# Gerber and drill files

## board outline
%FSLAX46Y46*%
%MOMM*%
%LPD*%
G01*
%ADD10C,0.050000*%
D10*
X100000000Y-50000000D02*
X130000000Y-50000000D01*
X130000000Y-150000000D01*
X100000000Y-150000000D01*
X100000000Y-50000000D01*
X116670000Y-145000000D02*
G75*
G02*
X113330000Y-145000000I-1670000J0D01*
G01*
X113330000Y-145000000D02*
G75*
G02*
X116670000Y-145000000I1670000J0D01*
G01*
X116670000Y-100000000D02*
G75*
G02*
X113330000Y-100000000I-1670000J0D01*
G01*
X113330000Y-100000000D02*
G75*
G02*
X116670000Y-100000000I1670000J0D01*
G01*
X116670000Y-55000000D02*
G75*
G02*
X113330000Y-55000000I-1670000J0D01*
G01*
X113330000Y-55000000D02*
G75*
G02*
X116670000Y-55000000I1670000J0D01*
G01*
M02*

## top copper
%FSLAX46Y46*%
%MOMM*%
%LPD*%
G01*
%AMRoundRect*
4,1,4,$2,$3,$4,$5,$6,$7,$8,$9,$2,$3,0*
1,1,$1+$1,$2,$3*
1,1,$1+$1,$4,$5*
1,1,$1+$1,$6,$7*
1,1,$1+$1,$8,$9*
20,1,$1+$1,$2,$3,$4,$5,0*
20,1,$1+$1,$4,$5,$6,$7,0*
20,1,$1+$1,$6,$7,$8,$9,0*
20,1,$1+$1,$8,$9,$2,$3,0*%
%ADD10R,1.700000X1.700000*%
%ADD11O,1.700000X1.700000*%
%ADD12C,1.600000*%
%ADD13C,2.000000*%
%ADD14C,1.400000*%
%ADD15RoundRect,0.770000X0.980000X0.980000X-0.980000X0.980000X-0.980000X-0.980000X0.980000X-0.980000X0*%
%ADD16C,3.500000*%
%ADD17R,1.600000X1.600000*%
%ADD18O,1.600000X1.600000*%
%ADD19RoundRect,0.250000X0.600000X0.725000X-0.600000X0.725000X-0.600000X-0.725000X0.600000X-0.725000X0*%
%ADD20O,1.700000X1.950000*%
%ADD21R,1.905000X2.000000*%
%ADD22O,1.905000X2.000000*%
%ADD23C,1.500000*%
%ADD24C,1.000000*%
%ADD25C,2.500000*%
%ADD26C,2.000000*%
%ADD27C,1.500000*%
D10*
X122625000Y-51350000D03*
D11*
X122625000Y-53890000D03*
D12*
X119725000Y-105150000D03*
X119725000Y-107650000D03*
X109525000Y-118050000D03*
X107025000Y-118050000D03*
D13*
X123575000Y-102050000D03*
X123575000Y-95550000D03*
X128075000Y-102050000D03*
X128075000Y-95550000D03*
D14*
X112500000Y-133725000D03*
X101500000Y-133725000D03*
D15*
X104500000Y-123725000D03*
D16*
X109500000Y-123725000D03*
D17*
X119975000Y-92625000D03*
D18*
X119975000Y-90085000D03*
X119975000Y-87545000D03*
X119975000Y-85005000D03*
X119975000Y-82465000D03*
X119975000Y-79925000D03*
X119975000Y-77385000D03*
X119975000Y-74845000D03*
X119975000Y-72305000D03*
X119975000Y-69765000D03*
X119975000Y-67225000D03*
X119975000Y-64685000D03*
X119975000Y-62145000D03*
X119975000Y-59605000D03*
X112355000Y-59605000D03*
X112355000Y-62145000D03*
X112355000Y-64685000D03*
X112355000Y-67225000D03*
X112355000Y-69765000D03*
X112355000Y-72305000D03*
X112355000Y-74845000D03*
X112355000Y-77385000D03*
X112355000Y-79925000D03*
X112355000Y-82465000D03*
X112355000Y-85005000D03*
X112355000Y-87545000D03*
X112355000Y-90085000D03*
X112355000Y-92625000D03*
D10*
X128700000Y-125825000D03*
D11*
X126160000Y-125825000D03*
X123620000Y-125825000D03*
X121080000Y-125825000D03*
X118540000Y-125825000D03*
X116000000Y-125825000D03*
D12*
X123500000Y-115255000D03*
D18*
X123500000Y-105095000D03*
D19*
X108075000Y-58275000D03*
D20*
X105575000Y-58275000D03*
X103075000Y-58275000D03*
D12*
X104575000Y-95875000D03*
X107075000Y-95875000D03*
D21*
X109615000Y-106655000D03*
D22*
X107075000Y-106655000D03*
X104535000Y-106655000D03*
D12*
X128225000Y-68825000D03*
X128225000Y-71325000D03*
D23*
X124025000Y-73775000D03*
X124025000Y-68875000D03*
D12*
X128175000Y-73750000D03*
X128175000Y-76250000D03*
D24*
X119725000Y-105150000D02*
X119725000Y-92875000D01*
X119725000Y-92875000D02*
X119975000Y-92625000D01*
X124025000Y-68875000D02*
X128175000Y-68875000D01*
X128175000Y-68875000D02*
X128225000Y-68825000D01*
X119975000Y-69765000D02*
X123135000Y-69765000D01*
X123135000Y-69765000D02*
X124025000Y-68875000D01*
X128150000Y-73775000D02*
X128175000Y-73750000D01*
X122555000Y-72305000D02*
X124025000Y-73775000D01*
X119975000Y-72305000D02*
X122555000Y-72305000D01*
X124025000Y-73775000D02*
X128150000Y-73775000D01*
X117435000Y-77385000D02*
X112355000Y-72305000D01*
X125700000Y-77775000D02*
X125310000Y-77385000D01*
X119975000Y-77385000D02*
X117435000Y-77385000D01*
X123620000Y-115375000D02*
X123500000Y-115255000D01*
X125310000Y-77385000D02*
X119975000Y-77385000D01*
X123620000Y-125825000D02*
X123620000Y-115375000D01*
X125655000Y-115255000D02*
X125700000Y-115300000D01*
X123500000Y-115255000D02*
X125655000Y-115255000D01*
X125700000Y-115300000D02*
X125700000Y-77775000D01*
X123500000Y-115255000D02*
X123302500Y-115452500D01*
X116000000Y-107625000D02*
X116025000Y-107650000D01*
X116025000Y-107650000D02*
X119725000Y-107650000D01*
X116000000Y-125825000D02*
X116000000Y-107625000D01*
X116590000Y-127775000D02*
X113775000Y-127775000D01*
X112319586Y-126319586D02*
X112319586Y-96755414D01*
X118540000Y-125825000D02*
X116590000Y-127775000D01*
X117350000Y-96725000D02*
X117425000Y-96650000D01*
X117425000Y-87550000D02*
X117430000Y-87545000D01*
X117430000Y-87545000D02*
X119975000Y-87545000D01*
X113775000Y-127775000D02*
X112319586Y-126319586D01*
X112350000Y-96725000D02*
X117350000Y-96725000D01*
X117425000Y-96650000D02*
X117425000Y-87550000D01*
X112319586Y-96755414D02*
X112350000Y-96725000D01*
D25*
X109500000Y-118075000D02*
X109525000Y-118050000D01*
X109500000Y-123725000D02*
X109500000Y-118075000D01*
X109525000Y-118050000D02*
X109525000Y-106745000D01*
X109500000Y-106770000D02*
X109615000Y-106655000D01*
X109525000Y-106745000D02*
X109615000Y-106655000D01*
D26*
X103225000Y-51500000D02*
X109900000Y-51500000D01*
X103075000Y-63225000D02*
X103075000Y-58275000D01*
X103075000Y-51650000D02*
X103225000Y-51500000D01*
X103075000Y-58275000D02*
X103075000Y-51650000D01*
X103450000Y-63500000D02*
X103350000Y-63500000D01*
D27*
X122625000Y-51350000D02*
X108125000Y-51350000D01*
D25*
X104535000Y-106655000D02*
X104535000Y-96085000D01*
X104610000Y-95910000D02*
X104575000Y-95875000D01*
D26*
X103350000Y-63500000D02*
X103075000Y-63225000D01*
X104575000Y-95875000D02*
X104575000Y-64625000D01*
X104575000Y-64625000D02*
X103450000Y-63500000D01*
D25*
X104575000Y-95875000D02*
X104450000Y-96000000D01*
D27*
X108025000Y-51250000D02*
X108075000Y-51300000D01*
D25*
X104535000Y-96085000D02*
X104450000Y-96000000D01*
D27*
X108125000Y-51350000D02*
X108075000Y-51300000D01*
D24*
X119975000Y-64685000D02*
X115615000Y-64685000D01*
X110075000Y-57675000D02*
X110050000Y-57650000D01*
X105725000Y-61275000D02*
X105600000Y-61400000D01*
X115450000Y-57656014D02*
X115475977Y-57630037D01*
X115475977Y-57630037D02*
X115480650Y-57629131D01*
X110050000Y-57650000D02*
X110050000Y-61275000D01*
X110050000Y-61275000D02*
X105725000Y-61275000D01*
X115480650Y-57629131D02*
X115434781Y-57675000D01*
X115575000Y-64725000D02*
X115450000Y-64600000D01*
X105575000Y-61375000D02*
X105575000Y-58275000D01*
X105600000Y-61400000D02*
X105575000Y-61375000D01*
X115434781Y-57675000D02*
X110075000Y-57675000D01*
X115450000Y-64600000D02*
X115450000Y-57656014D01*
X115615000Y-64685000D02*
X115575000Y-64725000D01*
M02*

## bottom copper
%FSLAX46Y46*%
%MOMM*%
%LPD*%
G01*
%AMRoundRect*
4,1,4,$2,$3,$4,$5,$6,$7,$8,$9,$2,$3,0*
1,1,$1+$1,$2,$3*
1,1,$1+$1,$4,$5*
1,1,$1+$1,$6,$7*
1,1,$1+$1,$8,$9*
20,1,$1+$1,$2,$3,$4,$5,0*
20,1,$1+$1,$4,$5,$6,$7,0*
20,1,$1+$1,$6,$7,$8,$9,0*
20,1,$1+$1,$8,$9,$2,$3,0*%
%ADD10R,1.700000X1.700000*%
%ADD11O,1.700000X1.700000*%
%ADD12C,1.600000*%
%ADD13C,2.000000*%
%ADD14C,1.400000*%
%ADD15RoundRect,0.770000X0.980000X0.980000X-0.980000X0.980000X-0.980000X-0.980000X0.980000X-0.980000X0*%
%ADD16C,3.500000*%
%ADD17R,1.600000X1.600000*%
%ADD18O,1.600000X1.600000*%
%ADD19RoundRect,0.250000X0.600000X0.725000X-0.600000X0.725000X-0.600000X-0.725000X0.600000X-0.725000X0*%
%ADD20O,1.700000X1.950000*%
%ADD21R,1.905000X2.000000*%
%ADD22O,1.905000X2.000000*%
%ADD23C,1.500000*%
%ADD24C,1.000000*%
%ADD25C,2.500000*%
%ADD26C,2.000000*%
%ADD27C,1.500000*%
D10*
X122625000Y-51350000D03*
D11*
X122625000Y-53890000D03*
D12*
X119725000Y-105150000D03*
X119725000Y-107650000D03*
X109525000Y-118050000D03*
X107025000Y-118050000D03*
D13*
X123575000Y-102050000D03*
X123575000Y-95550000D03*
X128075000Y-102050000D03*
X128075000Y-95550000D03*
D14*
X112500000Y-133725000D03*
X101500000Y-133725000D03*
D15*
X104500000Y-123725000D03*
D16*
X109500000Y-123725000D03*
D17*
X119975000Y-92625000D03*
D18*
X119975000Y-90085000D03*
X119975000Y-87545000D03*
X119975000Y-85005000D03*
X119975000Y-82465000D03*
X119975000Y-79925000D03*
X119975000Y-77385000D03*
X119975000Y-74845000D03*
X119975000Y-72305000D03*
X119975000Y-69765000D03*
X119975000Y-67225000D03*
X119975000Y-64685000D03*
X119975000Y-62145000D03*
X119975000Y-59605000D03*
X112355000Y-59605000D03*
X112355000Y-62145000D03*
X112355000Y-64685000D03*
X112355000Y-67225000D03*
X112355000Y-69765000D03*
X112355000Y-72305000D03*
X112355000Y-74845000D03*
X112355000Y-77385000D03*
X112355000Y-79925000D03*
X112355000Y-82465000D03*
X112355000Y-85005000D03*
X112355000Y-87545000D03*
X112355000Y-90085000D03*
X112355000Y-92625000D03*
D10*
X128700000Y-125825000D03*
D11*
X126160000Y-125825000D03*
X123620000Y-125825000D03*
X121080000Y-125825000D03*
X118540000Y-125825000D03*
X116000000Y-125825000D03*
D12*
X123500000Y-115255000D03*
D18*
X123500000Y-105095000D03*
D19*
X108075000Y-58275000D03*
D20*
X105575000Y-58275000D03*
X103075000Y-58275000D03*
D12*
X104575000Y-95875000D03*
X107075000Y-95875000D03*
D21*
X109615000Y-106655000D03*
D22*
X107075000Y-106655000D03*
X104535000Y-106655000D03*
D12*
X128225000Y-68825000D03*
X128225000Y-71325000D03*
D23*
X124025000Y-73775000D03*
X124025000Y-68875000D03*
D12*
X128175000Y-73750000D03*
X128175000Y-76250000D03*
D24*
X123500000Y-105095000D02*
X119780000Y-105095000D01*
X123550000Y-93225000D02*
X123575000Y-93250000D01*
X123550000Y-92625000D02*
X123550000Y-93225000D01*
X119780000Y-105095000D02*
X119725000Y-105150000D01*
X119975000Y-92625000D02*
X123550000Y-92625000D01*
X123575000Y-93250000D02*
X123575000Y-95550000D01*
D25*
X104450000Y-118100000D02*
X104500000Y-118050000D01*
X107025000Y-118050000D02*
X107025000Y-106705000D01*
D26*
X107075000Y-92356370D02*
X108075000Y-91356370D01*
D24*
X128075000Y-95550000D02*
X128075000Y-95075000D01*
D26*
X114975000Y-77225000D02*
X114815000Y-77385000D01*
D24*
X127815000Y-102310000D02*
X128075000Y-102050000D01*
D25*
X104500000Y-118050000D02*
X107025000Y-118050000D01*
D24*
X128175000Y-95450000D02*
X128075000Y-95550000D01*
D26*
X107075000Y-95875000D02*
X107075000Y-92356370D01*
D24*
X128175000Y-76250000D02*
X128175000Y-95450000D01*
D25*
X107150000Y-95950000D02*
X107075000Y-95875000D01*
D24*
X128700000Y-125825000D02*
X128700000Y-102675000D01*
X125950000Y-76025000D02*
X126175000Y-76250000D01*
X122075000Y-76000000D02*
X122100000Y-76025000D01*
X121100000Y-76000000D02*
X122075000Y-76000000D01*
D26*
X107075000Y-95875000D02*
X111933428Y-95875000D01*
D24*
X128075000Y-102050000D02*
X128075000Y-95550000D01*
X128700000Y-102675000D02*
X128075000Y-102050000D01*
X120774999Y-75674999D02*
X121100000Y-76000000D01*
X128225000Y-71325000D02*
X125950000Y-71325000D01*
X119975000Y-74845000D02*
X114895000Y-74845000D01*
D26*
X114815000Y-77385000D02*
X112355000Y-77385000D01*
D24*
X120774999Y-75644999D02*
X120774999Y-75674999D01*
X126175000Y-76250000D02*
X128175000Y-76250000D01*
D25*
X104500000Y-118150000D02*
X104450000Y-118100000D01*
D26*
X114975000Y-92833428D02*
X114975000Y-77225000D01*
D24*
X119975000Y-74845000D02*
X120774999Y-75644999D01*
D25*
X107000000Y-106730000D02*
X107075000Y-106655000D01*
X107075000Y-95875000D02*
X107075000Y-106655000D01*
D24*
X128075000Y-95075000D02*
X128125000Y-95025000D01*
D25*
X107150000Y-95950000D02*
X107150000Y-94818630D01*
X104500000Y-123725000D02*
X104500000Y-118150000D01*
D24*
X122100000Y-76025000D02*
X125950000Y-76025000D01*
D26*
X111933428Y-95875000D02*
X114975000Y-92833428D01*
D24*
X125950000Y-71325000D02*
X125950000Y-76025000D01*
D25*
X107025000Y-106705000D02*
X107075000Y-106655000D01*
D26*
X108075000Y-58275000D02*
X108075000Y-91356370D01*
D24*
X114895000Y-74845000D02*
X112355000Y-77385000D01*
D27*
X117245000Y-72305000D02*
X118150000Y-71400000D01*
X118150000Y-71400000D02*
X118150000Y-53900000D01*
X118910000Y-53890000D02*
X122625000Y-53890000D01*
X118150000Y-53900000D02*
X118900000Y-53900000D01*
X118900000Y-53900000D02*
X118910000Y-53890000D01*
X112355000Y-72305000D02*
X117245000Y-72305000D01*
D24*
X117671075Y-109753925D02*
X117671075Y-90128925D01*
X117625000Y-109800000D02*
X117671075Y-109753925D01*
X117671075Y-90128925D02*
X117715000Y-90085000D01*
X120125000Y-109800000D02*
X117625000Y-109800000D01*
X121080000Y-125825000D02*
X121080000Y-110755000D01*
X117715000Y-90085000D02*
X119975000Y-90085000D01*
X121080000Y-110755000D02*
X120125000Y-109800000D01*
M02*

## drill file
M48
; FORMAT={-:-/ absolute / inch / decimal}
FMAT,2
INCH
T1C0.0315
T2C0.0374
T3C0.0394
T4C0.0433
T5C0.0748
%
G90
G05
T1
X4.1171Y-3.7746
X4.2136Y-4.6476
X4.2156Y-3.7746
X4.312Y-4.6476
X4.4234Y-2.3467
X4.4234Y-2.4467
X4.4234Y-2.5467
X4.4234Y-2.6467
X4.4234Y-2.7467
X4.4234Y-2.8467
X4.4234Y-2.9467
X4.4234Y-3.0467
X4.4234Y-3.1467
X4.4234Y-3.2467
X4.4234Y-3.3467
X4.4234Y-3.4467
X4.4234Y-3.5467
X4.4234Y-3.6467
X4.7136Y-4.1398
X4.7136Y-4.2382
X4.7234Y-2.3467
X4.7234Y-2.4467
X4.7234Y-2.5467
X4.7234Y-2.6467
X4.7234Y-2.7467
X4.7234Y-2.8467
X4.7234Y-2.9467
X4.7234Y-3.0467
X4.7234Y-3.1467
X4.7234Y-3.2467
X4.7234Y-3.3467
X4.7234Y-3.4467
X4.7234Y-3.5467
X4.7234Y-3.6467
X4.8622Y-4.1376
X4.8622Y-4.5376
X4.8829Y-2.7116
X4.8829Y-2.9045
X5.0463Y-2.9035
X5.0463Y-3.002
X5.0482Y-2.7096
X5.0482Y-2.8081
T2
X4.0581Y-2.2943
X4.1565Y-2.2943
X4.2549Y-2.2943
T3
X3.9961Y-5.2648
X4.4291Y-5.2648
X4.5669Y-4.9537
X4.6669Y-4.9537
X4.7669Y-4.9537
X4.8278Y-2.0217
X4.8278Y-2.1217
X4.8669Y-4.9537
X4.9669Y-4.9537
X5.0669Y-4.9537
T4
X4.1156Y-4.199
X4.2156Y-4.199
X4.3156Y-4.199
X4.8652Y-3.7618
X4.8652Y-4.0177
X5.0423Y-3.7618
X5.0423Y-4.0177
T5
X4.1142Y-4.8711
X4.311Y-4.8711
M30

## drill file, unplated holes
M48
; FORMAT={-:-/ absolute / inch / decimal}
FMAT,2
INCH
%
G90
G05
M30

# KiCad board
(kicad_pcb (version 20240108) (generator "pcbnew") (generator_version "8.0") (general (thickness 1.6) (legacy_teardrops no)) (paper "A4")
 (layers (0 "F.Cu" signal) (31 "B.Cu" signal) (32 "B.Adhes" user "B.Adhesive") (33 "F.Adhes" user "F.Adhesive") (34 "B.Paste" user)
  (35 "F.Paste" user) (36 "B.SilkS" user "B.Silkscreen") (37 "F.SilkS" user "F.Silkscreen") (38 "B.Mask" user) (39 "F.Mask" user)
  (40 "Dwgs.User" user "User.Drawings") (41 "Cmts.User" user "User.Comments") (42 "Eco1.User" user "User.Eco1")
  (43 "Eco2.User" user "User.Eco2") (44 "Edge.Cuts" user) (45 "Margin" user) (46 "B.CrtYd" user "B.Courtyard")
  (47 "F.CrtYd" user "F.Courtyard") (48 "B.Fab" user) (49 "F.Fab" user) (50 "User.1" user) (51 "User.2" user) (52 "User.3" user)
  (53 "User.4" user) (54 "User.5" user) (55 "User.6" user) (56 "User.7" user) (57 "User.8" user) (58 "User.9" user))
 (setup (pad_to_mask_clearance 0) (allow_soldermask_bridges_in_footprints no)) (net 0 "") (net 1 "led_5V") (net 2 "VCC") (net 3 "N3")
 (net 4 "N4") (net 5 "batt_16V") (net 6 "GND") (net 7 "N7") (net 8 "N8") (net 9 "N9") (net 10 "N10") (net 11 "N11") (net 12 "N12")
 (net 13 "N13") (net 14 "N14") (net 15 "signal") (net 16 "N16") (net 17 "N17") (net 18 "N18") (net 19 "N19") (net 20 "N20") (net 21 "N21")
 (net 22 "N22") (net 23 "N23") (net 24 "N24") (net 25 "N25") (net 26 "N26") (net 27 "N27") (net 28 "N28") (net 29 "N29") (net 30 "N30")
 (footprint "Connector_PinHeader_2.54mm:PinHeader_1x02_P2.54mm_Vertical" (layer "F.Cu") (at 122.625 51.35)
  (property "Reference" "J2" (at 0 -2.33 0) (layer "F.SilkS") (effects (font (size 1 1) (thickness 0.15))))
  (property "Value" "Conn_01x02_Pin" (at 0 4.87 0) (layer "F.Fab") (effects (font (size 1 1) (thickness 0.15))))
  (pad "1" thru_hole rect (at 0 0) (size 1.7 1.7) (drill 1) (layers "*.Cu" "*.Mask") (remove_unused_layers no) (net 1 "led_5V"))
  (pad "2" thru_hole oval (at 0 2.54) (size 1.7 1.7) (drill 1) (layers "*.Cu" "*.Mask") (remove_unused_layers no) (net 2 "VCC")))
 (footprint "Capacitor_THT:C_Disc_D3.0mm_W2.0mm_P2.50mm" (layer "F.Cu") (at 119.725 105.15 -90)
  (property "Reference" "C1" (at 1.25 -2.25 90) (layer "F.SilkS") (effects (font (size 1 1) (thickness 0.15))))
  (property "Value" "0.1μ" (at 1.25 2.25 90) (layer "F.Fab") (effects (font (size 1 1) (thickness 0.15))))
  (pad "1" thru_hole circle (at 0 0 270) (size 1.6 1.6) (drill 0.8) (layers "*.Cu" "*.Mask") (remove_unused_layers no) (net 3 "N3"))
  (pad "2" thru_hole circle (at 2.5 0 270) (size 1.6 1.6) (drill 0.8) (layers "*.Cu" "*.Mask") (remove_unused_layers no) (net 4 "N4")))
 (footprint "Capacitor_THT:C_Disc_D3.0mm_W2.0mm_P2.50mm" (layer "F.Cu") (at 109.525 118.05 180)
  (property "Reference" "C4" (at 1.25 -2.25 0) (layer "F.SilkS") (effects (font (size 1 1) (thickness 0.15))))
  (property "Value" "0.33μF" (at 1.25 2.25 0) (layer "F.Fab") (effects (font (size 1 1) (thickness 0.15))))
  (pad "1" thru_hole circle (at 0 0 180) (size 1.6 1.6) (drill 0.8) (layers "*.Cu" "*.Mask") (remove_unused_layers no) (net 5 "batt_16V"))
  (pad "2" thru_hole circle (at 2.5 0 180) (size 1.6 1.6) (drill 0.8) (layers "*.Cu" "*.Mask") (remove_unused_layers no) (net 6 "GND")))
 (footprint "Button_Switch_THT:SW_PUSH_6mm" (layer "F.Cu") (at 123.575 102.05 90)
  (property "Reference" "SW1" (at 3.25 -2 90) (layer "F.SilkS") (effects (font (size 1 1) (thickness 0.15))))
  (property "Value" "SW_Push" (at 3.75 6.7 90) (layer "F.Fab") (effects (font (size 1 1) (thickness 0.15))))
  (pad "1" thru_hole circle (at 0 0 180) (size 2 2) (drill 1.1) (layers "*.Cu" "*.Mask") (remove_unused_layers no) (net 3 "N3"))
  (pad "1" thru_hole circle (at 6.5 0 180) (size 2 2) (drill 1.1) (layers "*.Cu" "*.Mask") (remove_unused_layers no) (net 3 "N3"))
  (pad "2" thru_hole circle (at 0 4.5 180) (size 2 2) (drill 1.1) (layers "*.Cu" "*.Mask") (remove_unused_layers no) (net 6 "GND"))
  (pad "2" thru_hole circle (at 6.5 4.5 180) (size 2 2) (drill 1.1) (layers "*.Cu" "*.Mask") (remove_unused_layers no) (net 6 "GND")))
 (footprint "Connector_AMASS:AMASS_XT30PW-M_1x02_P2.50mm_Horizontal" (layer "F.Cu") (at 104.5 123.725 180)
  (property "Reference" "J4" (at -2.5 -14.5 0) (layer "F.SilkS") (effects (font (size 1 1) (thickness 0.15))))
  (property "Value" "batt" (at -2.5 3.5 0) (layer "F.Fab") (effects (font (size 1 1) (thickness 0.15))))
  (pad "" thru_hole circle (at -8 -10 180) (size 1.4 1.4) (drill 1) (layers "*.Cu" "*.Mask") (remove_unused_layers no))
  (pad "" thru_hole circle (at 3 -10 180) (size 1.4 1.4) (drill 1) (layers "*.Cu" "*.Mask") (remove_unused_layers no))
  (pad "1" thru_hole roundrect (at 0 0 180) (size 3.5 3.5) (drill 1.9) (layers "*.Cu" "*.Mask") (remove_unused_layers no)
   (roundrect_rratio 0.22) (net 6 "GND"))
  (pad "2" thru_hole circle (at -5 0 180) (size 3.5 3.5) (drill 1.9) (layers "*.Cu" "*.Mask") (remove_unused_layers no) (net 5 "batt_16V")))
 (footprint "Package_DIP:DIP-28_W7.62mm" (layer "F.Cu") (at 119.975 92.625 180)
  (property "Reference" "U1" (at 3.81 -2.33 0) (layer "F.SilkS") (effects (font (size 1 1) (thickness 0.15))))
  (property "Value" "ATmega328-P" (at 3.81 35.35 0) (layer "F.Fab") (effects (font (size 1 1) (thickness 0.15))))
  (pad "1" thru_hole rect (at 0 0 180) (size 1.6 1.6) (drill 0.8) (layers "*.Cu" "*.Mask") (remove_unused_layers no) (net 3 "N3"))
  (pad "2" thru_hole oval (at 0 2.54 180) (size 1.6 1.6) (drill 0.8) (layers "*.Cu" "*.Mask") (remove_unused_layers no) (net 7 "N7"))
  (pad "3" thru_hole oval (at 0 5.08 180) (size 1.6 1.6) (drill 0.8) (layers "*.Cu" "*.Mask") (remove_unused_layers no) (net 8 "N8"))
  (pad "4" thru_hole oval (at 0 7.62 180) (size 1.6 1.6) (drill 0.8) (layers "*.Cu" "*.Mask") (remove_unused_layers no) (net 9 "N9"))
  (pad "5" thru_hole oval (at 0 10.16 180) (size 1.6 1.6) (drill 0.8) (layers "*.Cu" "*.Mask") (remove_unused_layers no) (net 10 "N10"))
  (pad "6" thru_hole oval (at 0 12.7 180) (size 1.6 1.6) (drill 0.8) (layers "*.Cu" "*.Mask") (remove_unused_layers no) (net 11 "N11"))
  (pad "7" thru_hole oval (at 0 15.24 180) (size 1.6 1.6) (drill 0.8) (layers "*.Cu" "*.Mask") (remove_unused_layers no) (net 2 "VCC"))
  (pad "8" thru_hole oval (at 0 17.78 180) (size 1.6 1.6) (drill 0.8) (layers "*.Cu" "*.Mask") (remove_unused_layers no) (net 6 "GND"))
  (pad "9" thru_hole oval (at 0 20.32 180) (size 1.6 1.6) (drill 0.8) (layers "*.Cu" "*.Mask") (remove_unused_layers no) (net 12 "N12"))
  (pad "10" thru_hole oval (at 0 22.86 180) (size 1.6 1.6) (drill 0.8) (layers "*.Cu" "*.Mask") (remove_unused_layers no) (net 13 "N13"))
  (pad "11" thru_hole oval (at 0 25.4 180) (size 1.6 1.6) (drill 0.8) (layers "*.Cu" "*.Mask") (remove_unused_layers no) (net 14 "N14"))
  (pad "12" thru_hole oval (at 0 27.94 180) (size 1.6 1.6) (drill 0.8) (layers "*.Cu" "*.Mask") (remove_unused_layers no) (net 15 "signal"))
  (pad "13" thru_hole oval (at 0 30.48 180) (size 1.6 1.6) (drill 0.8) (layers "*.Cu" "*.Mask") (remove_unused_layers no) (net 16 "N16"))
  (pad "14" thru_hole oval (at 0 33.02 180) (size 1.6 1.6) (drill 0.8) (layers "*.Cu" "*.Mask") (remove_unused_layers no) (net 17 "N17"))
  (pad "15" thru_hole oval (at 7.62 33.02 180) (size 1.6 1.6) (drill 0.8) (layers "*.Cu" "*.Mask") (remove_unused_layers no) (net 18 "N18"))
  (pad "16" thru_hole oval (at 7.62 30.48 180) (size 1.6 1.6) (drill 0.8) (layers "*.Cu" "*.Mask") (remove_unused_layers no) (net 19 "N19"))
  (pad "17" thru_hole oval (at 7.62 27.94 180) (size 1.6 1.6) (drill 0.8) (layers "*.Cu" "*.Mask") (remove_unused_layers no) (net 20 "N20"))
  (pad "18" thru_hole oval (at 7.62 25.4 180) (size 1.6 1.6) (drill 0.8) (layers "*.Cu" "*.Mask") (remove_unused_layers no) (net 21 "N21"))
  (pad "19" thru_hole oval (at 7.62 22.86 180) (size 1.6 1.6) (drill 0.8) (layers "*.Cu" "*.Mask") (remove_unused_layers no) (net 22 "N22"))
  (pad "20" thru_hole oval (at 7.62 20.32 180) (size 1.6 1.6) (drill 0.8) (layers "*.Cu" "*.Mask") (remove_unused_layers no) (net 2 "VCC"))
  (pad "21" thru_hole oval (at 7.62 17.78 180) (size 1.6 1.6) (drill 0.8) (layers "*.Cu" "*.Mask") (remove_unused_layers no) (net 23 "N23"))
  (pad "22" thru_hole oval (at 7.62 15.24 180) (size 1.6 1.6) (drill 0.8) (layers "*.Cu" "*.Mask") (remove_unused_layers no) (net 6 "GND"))
  (pad "23" thru_hole oval (at 7.62 12.7 180) (size 1.6 1.6) (drill 0.8) (layers "*.Cu" "*.Mask") (remove_unused_layers no) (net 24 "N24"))
  (pad "24" thru_hole oval (at 7.62 10.16 180) (size 1.6 1.6) (drill 0.8) (layers "*.Cu" "*.Mask") (remove_unused_layers no) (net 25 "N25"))
  (pad "25" thru_hole oval (at 7.62 7.62 180) (size 1.6 1.6) (drill 0.8) (layers "*.Cu" "*.Mask") (remove_unused_layers no) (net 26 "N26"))
  (pad "26" thru_hole oval (at 7.62 5.08 180) (size 1.6 1.6) (drill 0.8) (layers "*.Cu" "*.Mask") (remove_unused_layers no) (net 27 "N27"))
  (pad "27" thru_hole oval (at 7.62 2.54 180) (size 1.6 1.6) (drill 0.8) (layers "*.Cu" "*.Mask") (remove_unused_layers no) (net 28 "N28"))
  (pad "28" thru_hole oval (at 7.62 0 180) (size 1.6 1.6) (drill 0.8) (layers "*.Cu" "*.Mask") (remove_unused_layers no) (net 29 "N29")))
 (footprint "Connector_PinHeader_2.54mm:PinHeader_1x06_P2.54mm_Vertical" (layer "F.Cu") (at 128.7 125.825 -90)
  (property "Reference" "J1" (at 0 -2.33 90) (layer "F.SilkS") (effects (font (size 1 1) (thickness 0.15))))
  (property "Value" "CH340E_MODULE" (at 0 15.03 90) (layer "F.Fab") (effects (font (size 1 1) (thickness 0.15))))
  (pad "1" thru_hole rect (at 0 0 270) (size 1.7 1.7) (drill 1) (layers "*.Cu" "*.Mask") (remove_unused_layers no) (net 6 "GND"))
  (pad "2" thru_hole oval (at 0 2.54 270) (size 1.7 1.7) (drill 1) (layers "*.Cu" "*.Mask") (remove_unused_layers no) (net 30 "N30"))
  (pad "3" thru_hole oval (at 0 5.08 270) (size 1.7 1.7) (drill 1) (layers "*.Cu" "*.Mask") (remove_unused_layers no) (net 2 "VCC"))
  (pad "4" thru_hole oval (at 0 7.62 270) (size 1.7 1.7) (drill 1) (layers "*.Cu" "*.Mask") (remove_unused_layers no) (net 7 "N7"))
  (pad "5" thru_hole oval (at 0 10.16 270) (size 1.7 1.7) (drill 1) (layers "*.Cu" "*.Mask") (remove_unused_layers no) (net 8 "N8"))
  (pad "6" thru_hole oval (at 0 12.7 270) (size 1.7 1.7) (drill 1) (layers "*.Cu" "*.Mask") (remove_unused_layers no) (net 4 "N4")))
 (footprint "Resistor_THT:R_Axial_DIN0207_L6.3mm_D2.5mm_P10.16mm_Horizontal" (layer "F.Cu") (at 123.5 115.255 90)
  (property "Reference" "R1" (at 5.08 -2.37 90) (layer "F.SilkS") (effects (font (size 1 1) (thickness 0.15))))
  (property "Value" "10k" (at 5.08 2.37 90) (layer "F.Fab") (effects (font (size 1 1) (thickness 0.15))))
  (pad "1" thru_hole circle (at 0 0 90) (size 1.6 1.6) (drill 0.8) (layers "*.Cu" "*.Mask") (remove_unused_layers no) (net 2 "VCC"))
  (pad "2" thru_hole oval (at 10.16 0 90) (size 1.6 1.6) (drill 0.8) (layers "*.Cu" "*.Mask") (remove_unused_layers no) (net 3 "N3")))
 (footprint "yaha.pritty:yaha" (layer "F.Cu") (at 108.4 75.8 -90)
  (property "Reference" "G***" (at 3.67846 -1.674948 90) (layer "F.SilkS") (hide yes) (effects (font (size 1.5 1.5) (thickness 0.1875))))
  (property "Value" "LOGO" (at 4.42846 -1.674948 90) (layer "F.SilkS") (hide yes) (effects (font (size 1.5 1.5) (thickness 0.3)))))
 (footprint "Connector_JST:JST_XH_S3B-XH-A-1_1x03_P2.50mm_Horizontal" (layer "F.Cu") (at 108.075 58.275 180)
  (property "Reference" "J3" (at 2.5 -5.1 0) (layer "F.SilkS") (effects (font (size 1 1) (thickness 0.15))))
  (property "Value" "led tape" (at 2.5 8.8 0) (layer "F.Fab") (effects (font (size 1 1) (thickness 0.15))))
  (pad "1" thru_hole roundrect (at 0 0 180) (size 1.7 1.95) (drill 0.95) (layers "*.Cu" "*.Mask") (remove_unused_layers no)
   (roundrect_rratio 0.147059) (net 6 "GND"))
  (pad "2" thru_hole oval (at 2.5 0 180) (size 1.7 1.95) (drill 0.95) (layers "*.Cu" "*.Mask") (remove_unused_layers no) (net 15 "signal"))
  (pad "3" thru_hole oval (at 5 0 180) (size 1.7 1.95) (drill 0.95) (layers "*.Cu" "*.Mask") (remove_unused_layers no) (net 1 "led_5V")))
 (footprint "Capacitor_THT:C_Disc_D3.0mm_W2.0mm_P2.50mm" (layer "F.Cu") (at 104.575 95.875)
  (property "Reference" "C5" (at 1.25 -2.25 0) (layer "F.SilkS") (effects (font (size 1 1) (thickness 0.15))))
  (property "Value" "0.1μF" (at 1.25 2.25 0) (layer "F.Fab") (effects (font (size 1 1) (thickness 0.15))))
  (pad "1" thru_hole circle (at 0 0) (size 1.6 1.6) (drill 0.8) (layers "*.Cu" "*.Mask") (remove_unused_layers no) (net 1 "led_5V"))
  (pad "2" thru_hole circle (at 2.5 0) (size 1.6 1.6) (drill 0.8) (layers "*.Cu" "*.Mask") (remove_unused_layers no) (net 6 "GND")))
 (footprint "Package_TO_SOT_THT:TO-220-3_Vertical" (layer "F.Cu") (at 109.615 106.655 180)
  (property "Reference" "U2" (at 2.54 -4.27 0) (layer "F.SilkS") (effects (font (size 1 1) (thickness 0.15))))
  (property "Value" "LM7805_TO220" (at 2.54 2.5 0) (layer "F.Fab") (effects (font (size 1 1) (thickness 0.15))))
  (pad "1" thru_hole rect (at 0 0 180) (size 1.905 2) (drill 1.1) (layers "*.Cu" "*.Mask") (remove_unused_layers no) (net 5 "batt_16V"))
  (pad "2" thru_hole oval (at 2.54 0 180) (size 1.905 2) (drill 1.1) (layers "*.Cu" "*.Mask") (remove_unused_layers no) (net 6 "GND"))
  (pad "3" thru_hole oval (at 5.08 0 180) (size 1.905 2) (drill 1.1) (layers "*.Cu" "*.Mask") (remove_unused_layers no) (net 1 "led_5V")))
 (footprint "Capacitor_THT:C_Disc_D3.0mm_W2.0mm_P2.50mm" (layer "F.Cu") (at 128.225 68.825 -90)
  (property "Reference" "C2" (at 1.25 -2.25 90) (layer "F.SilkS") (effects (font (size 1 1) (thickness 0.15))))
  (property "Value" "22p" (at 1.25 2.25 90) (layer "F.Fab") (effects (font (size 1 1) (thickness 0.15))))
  (pad "1" thru_hole circle (at 0 0 270) (size 1.6 1.6) (drill 0.8) (layers "*.Cu" "*.Mask") (remove_unused_layers no) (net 13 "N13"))
  (pad "2" thru_hole circle (at 2.5 0 270) (size 1.6 1.6) (drill 0.8) (layers "*.Cu" "*.Mask") (remove_unused_layers no) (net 6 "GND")))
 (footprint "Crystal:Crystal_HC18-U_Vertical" (layer "F.Cu") (at 124.025 73.775 90)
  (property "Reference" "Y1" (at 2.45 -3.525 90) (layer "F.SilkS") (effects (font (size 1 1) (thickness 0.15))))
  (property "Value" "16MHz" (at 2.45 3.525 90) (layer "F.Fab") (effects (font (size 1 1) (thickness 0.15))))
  (pad "1" thru_hole circle (at 0 0 90) (size 1.5 1.5) (drill 0.8) (layers "*.Cu" "*.Mask") (remove_unused_layers no) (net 12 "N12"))
  (pad "2" thru_hole circle (at 4.9 0 90) (size 1.5 1.5) (drill 0.8) (layers "*.Cu" "*.Mask") (remove_unused_layers no) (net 13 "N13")))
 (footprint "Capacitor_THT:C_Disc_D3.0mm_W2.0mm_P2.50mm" (layer "F.Cu") (at 128.175 73.75 -90)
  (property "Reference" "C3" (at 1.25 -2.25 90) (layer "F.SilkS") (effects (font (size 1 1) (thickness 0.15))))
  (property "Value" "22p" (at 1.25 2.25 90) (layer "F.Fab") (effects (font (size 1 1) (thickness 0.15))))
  (pad "1" thru_hole circle (at 0 0 270) (size 1.6 1.6) (drill 0.8) (layers "*.Cu" "*.Mask") (remove_unused_layers no) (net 12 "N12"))
  (pad "2" thru_hole circle (at 2.5 0 270) (size 1.6 1.6) (drill 0.8) (layers "*.Cu" "*.Mask") (remove_unused_layers no) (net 6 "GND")))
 (gr_rect (start 100 50) (end 130 150) (stroke (width 0.05) (type default)) (fill none) (layer "Edge.Cuts"))
 (gr_circle (center 115 145) (end 116.67 145) (stroke (width 0.05) (type default)) (fill none) (layer "Edge.Cuts"))
 (gr_circle (center 115 100) (end 116.67 100) (stroke (width 0.05) (type default)) (fill none) (layer "Edge.Cuts"))
 (gr_circle (center 115 55) (end 116.67 55) (stroke (width 0.05) (type default)) (fill none) (layer "Edge.Cuts"))
 (segment (start 119.725 105.15) (end 119.725 92.875) (width 1) (layer "F.Cu") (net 3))
 (segment (start 119.725 92.875) (end 119.975 92.625) (width 1) (layer "F.Cu") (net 3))
 (segment (start 123.5 105.095) (end 119.78 105.095) (width 1) (layer "B.Cu") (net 3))
 (segment (start 123.55 93.225) (end 123.575 93.25) (width 1) (layer "B.Cu") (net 3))
 (segment (start 123.55 92.625) (end 123.55 93.225) (width 1) (layer "B.Cu") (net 3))
 (segment (start 119.78 105.095) (end 119.725 105.15) (width 1) (layer "B.Cu") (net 3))
 (segment (start 119.975 92.625) (end 123.55 92.625) (width 1) (layer "B.Cu") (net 3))
 (segment (start 123.575 93.25) (end 123.575 95.55) (width 1) (layer "B.Cu") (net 3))
 (segment (start 124.025 68.875) (end 128.175 68.875) (width 1) (layer "F.Cu") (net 13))
 (segment (start 128.175 68.875) (end 128.225 68.825) (width 1) (layer "F.Cu") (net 13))
 (segment (start 119.975 69.765) (end 123.135 69.765) (width 1) (layer "F.Cu") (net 13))
 (segment (start 123.135 69.765) (end 124.025 68.875) (width 1) (layer "F.Cu") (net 13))
 (segment (start 104.45 118.1) (end 104.5 118.05) (width 2.5) (layer "B.Cu") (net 6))
 (segment (start 107.025 118.05) (end 107.025 106.705) (width 2.5) (layer "B.Cu") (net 6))
 (segment (start 107.075 92.35637) (end 108.075 91.35637) (width 2) (layer "B.Cu") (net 6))
 (segment (start 128.075 95.55) (end 128.075 95.075) (width 1) (layer "B.Cu") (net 6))
 (segment (start 114.975 77.225) (end 114.815 77.385) (width 2) (layer "B.Cu") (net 6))
 (segment (start 127.815 102.31) (end 128.075 102.05) (width 1) (layer "B.Cu") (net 6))
 (segment (start 104.5 118.05) (end 107.025 118.05) (width 2.5) (layer "B.Cu") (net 6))
 (segment (start 128.175 95.45) (end 128.075 95.55) (width 1) (layer "B.Cu") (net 6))
 (segment (start 107.075 95.875) (end 107.075 92.35637) (width 2) (layer "B.Cu") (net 6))
 (segment (start 128.175 76.25) (end 128.175 95.45) (width 1) (layer "B.Cu") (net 6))
 (segment (start 107.15 95.95) (end 107.075 95.875) (width 2.5) (layer "B.Cu") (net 6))
 (segment (start 128.7 125.825) (end 128.7 102.675) (width 1) (layer "B.Cu") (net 6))
 (segment (start 125.95 76.025) (end 126.175 76.25) (width 1) (layer "B.Cu") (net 6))
 (segment (start 122.075 76) (end 122.1 76.025) (width 1) (layer "B.Cu") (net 6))
 (segment (start 121.1 76) (end 122.075 76) (width 1) (layer "B.Cu") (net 6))
 (segment (start 107.075 95.875) (end 111.933428 95.875) (width 2) (layer "B.Cu") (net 6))
 (segment (start 128.075 102.05) (end 128.075 95.55) (width 1) (layer "B.Cu") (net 6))
 (segment (start 128.7 102.675) (end 128.075 102.05) (width 1) (layer "B.Cu") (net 6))
 (segment (start 120.774999 75.674999) (end 121.1 76) (width 1) (layer "B.Cu") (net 6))
 (segment (start 128.225 71.325) (end 125.95 71.325) (width 1) (layer "B.Cu") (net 6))
 (segment (start 119.975 74.845) (end 114.895 74.845) (width 1) (layer "B.Cu") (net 6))
 (segment (start 114.815 77.385) (end 112.355 77.385) (width 2) (layer "B.Cu") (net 6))
 (segment (start 120.774999 75.644999) (end 120.774999 75.674999) (width 1) (layer "B.Cu") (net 6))
 (segment (start 126.175 76.25) (end 128.175 76.25) (width 1) (layer "B.Cu") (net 6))
 (segment (start 104.5 118.15) (end 104.45 118.1) (width 2.5) (layer "B.Cu") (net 6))
 (segment (start 114.975 92.833428) (end 114.975 77.225) (width 2) (layer "B.Cu") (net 6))
 (segment (start 119.975 74.845) (end 120.774999 75.644999) (width 1) (layer "B.Cu") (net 6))
 (segment (start 107 106.73) (end 107.075 106.655) (width 2.5) (layer "B.Cu") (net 6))
 (segment (start 107.075 95.875) (end 107.075 106.655) (width 2.5) (layer "B.Cu") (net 6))
 (segment (start 128.075 95.075) (end 128.125 95.025) (width 1) (layer "B.Cu") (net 6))
 (segment (start 107.15 95.95) (end 107.15 94.81863) (width 2.5) (layer "B.Cu") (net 6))
 (segment (start 104.5 123.725) (end 104.5 118.15) (width 2.5) (layer "B.Cu") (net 6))
 (segment (start 122.1 76.025) (end 125.95 76.025) (width 1) (layer "B.Cu") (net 6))
 (segment (start 111.933428 95.875) (end 114.975 92.833428) (width 2) (layer "B.Cu") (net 6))
 (segment (start 125.95 71.325) (end 125.95 76.025) (width 1) (layer "B.Cu") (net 6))
 (segment (start 107.025 106.705) (end 107.075 106.655) (width 2.5) (layer "B.Cu") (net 6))
 (segment (start 108.075 58.275) (end 108.075 91.35637) (width 2) (layer "B.Cu") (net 6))
 (segment (start 114.895 74.845) (end 112.355 77.385) (width 1) (layer "B.Cu") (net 6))
 (segment (start 128.15 73.775) (end 128.175 73.75) (width 1) (layer "F.Cu") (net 12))
 (segment (start 122.555 72.305) (end 124.025 73.775) (width 1) (layer "F.Cu") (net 12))
 (segment (start 119.975 72.305) (end 122.555 72.305) (width 1) (layer "F.Cu") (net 12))
 (segment (start 124.025 73.775) (end 128.15 73.775) (width 1) (layer "F.Cu") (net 12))
 (segment (start 117.435 77.385) (end 112.355 72.305) (width 1) (layer "F.Cu") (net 2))
 (segment (start 125.7 77.775) (end 125.31 77.385) (width 1) (layer "F.Cu") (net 2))
 (segment (start 119.975 77.385) (end 117.435 77.385) (width 1) (layer "F.Cu") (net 2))
 (segment (start 123.62 115.375) (end 123.5 115.255) (width 1) (layer "F.Cu") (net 2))
 (segment (start 125.31 77.385) (end 119.975 77.385) (width 1) (layer "F.Cu") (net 2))
 (segment (start 123.62 125.825) (end 123.62 115.375) (width 1) (layer "F.Cu") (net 2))
 (segment (start 125.655 115.255) (end 125.7 115.3) (width 1) (layer "F.Cu") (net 2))
 (segment (start 123.5 115.255) (end 125.655 115.255) (width 1) (layer "F.Cu") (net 2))
 (segment (start 125.7 115.3) (end 125.7 77.775) (width 1) (layer "F.Cu") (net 2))
 (segment (start 123.5 115.255) (end 123.3025 115.4525) (width 1) (layer "F.Cu") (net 2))
 (segment (start 117.245 72.305) (end 118.15 71.4) (width 1.5) (layer "B.Cu") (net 2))
 (segment (start 118.15 71.4) (end 118.15 53.9) (width 1.5) (layer "B.Cu") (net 2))
 (segment (start 118.91 53.89) (end 122.625 53.89) (width 1.5) (layer "B.Cu") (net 2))
 (segment (start 118.15 53.9) (end 118.9 53.9) (width 1.5) (layer "B.Cu") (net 2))
 (segment (start 118.9 53.9) (end 118.91 53.89) (width 1.5) (layer "B.Cu") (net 2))
 (segment (start 112.355 72.305) (end 117.245 72.305) (width 1.5) (layer "B.Cu") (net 2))
 (segment (start 116 107.625) (end 116.025 107.65) (width 1) (layer "F.Cu") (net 4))
 (segment (start 116.025 107.65) (end 119.725 107.65) (width 1) (layer "F.Cu") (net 4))
 (segment (start 116 125.825) (end 116 107.625) (width 1) (layer "F.Cu") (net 4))
 (segment (start 116.59 127.775) (end 113.775 127.775) (width 1) (layer "F.Cu") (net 8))
 (segment (start 112.319586 126.319586) (end 112.319586 96.755414) (width 1) (layer "F.Cu") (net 8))
 (segment (start 118.54 125.825) (end 116.59 127.775) (width 1) (layer "F.Cu") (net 8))
 (segment (start 117.35 96.725) (end 117.425 96.65) (width 1) (layer "F.Cu") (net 8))
 (segment (start 117.425 87.55) (end 117.43 87.545) (width 1) (layer "F.Cu") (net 8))
 (segment (start 117.43 87.545) (end 119.975 87.545) (width 1) (layer "F.Cu") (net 8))
 (segment (start 113.775 127.775) (end 112.319586 126.319586) (width 1) (layer "F.Cu") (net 8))
 (segment (start 112.35 96.725) (end 117.35 96.725) (width 1) (layer "F.Cu") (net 8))
 (segment (start 117.425 96.65) (end 117.425 87.55) (width 1) (layer "F.Cu") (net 8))
 (segment (start 112.319586 96.755414) (end 112.35 96.725) (width 1) (layer "F.Cu") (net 8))
 (segment (start 117.671075 109.753925) (end 117.671075 90.128925) (width 1) (layer "B.Cu") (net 7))
 (segment (start 117.625 109.8) (end 117.671075 109.753925) (width 1) (layer "B.Cu") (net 7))
 (segment (start 117.671075 90.128925) (end 117.715 90.085) (width 1) (layer "B.Cu") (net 7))
 (segment (start 120.125 109.8) (end 117.625 109.8) (width 1) (layer "B.Cu") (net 7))
 (segment (start 121.08 125.825) (end 121.08 110.755) (width 1) (layer "B.Cu") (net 7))
 (segment (start 117.715 90.085) (end 119.975 90.085) (width 1) (layer "B.Cu") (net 7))
 (segment (start 121.08 110.755) (end 120.125 109.8) (width 1) (layer "B.Cu") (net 7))
 (segment (start 109.5 118.075) (end 109.525 118.05) (width 2.5) (layer "F.Cu") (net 5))
 (segment (start 109.5 123.725) (end 109.5 118.075) (width 2.5) (layer "F.Cu") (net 5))
 (segment (start 109.525 118.05) (end 109.525 106.745) (width 2.5) (layer "F.Cu") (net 5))
 (segment (start 109.5 106.77) (end 109.615 106.655) (width 2.5) (layer "F.Cu") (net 5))
 (segment (start 109.525 106.745) (end 109.615 106.655) (width 2.5) (layer "F.Cu") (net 5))
 (segment (start 103.225 51.5) (end 109.9 51.5) (width 2) (layer "F.Cu") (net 1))
 (segment (start 103.075 63.225) (end 103.075 58.275) (width 2) (layer "F.Cu") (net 1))
 (segment (start 103.075 51.65) (end 103.225 51.5) (width 2) (layer "F.Cu") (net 1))
 (segment (start 103.075 58.275) (end 103.075 51.65) (width 2) (layer "F.Cu") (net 1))
 (segment (start 103.45 63.5) (end 103.35 63.5) (width 2) (layer "F.Cu") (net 1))
 (segment (start 122.625 51.35) (end 108.125 51.35) (width 1.5) (layer "F.Cu") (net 1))
 (segment (start 104.535 106.655) (end 104.535 96.085) (width 2.5) (layer "F.Cu") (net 1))
 (segment (start 104.61 95.91) (end 104.575 95.875) (width 2.5) (layer "F.Cu") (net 1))
 (segment (start 103.35 63.5) (end 103.075 63.225) (width 2) (layer "F.Cu") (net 1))
 (segment (start 104.575 95.875) (end 104.575 64.625) (width 2) (layer "F.Cu") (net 1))
 (segment (start 104.575 64.625) (end 103.45 63.5) (width 2) (layer "F.Cu") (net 1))
 (segment (start 104.575 95.875) (end 104.45 96) (width 2.5) (layer "F.Cu") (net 1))
 (segment (start 108.025 51.25) (end 108.075 51.3) (width 1.5) (layer "F.Cu") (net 1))
 (segment (start 104.535 96.085) (end 104.45 96) (width 2.5) (layer "F.Cu") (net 1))
 (segment (start 108.125 51.35) (end 108.075 51.3) (width 1.5) (layer "F.Cu") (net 1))
 (segment (start 119.975 64.685) (end 115.615 64.685) (width 1) (layer "F.Cu") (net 15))
 (segment (start 110.075 57.675) (end 110.05 57.65) (width 1) (layer "F.Cu") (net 15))
 (segment (start 105.725 61.275) (end 105.6 61.4) (width 1) (layer "F.Cu") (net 15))
 (segment (start 115.45 57.656014) (end 115.475977 57.630037) (width 1) (layer "F.Cu") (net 15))
 (segment (start 115.475977 57.630037) (end 115.48065 57.629131) (width 1) (layer "F.Cu") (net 15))
 (segment (start 110.05 57.65) (end 110.05 61.275) (width 1) (layer "F.Cu") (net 15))
 (segment (start 110.05 61.275) (end 105.725 61.275) (width 1) (layer "F.Cu") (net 15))
 (segment (start 115.48065 57.629131) (end 115.434781 57.675) (width 1) (layer "F.Cu") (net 15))
 (segment (start 115.575 64.725) (end 115.45 64.6) (width 1) (layer "F.Cu") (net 15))
 (segment (start 105.575 61.375) (end 105.575 58.275) (width 1) (layer "F.Cu") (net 15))
 (segment (start 105.6 61.4) (end 105.575 61.375) (width 1) (layer "F.Cu") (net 15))
 (segment (start 115.434781 57.675) (end 110.075 57.675) (width 1) (layer "F.Cu") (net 15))
 (segment (start 115.45 64.6) (end 115.45 57.656014) (width 1) (layer "F.Cu") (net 15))
 (segment (start 115.615 64.685) (end 115.575 64.725) (width 1) (layer "F.Cu") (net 15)))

